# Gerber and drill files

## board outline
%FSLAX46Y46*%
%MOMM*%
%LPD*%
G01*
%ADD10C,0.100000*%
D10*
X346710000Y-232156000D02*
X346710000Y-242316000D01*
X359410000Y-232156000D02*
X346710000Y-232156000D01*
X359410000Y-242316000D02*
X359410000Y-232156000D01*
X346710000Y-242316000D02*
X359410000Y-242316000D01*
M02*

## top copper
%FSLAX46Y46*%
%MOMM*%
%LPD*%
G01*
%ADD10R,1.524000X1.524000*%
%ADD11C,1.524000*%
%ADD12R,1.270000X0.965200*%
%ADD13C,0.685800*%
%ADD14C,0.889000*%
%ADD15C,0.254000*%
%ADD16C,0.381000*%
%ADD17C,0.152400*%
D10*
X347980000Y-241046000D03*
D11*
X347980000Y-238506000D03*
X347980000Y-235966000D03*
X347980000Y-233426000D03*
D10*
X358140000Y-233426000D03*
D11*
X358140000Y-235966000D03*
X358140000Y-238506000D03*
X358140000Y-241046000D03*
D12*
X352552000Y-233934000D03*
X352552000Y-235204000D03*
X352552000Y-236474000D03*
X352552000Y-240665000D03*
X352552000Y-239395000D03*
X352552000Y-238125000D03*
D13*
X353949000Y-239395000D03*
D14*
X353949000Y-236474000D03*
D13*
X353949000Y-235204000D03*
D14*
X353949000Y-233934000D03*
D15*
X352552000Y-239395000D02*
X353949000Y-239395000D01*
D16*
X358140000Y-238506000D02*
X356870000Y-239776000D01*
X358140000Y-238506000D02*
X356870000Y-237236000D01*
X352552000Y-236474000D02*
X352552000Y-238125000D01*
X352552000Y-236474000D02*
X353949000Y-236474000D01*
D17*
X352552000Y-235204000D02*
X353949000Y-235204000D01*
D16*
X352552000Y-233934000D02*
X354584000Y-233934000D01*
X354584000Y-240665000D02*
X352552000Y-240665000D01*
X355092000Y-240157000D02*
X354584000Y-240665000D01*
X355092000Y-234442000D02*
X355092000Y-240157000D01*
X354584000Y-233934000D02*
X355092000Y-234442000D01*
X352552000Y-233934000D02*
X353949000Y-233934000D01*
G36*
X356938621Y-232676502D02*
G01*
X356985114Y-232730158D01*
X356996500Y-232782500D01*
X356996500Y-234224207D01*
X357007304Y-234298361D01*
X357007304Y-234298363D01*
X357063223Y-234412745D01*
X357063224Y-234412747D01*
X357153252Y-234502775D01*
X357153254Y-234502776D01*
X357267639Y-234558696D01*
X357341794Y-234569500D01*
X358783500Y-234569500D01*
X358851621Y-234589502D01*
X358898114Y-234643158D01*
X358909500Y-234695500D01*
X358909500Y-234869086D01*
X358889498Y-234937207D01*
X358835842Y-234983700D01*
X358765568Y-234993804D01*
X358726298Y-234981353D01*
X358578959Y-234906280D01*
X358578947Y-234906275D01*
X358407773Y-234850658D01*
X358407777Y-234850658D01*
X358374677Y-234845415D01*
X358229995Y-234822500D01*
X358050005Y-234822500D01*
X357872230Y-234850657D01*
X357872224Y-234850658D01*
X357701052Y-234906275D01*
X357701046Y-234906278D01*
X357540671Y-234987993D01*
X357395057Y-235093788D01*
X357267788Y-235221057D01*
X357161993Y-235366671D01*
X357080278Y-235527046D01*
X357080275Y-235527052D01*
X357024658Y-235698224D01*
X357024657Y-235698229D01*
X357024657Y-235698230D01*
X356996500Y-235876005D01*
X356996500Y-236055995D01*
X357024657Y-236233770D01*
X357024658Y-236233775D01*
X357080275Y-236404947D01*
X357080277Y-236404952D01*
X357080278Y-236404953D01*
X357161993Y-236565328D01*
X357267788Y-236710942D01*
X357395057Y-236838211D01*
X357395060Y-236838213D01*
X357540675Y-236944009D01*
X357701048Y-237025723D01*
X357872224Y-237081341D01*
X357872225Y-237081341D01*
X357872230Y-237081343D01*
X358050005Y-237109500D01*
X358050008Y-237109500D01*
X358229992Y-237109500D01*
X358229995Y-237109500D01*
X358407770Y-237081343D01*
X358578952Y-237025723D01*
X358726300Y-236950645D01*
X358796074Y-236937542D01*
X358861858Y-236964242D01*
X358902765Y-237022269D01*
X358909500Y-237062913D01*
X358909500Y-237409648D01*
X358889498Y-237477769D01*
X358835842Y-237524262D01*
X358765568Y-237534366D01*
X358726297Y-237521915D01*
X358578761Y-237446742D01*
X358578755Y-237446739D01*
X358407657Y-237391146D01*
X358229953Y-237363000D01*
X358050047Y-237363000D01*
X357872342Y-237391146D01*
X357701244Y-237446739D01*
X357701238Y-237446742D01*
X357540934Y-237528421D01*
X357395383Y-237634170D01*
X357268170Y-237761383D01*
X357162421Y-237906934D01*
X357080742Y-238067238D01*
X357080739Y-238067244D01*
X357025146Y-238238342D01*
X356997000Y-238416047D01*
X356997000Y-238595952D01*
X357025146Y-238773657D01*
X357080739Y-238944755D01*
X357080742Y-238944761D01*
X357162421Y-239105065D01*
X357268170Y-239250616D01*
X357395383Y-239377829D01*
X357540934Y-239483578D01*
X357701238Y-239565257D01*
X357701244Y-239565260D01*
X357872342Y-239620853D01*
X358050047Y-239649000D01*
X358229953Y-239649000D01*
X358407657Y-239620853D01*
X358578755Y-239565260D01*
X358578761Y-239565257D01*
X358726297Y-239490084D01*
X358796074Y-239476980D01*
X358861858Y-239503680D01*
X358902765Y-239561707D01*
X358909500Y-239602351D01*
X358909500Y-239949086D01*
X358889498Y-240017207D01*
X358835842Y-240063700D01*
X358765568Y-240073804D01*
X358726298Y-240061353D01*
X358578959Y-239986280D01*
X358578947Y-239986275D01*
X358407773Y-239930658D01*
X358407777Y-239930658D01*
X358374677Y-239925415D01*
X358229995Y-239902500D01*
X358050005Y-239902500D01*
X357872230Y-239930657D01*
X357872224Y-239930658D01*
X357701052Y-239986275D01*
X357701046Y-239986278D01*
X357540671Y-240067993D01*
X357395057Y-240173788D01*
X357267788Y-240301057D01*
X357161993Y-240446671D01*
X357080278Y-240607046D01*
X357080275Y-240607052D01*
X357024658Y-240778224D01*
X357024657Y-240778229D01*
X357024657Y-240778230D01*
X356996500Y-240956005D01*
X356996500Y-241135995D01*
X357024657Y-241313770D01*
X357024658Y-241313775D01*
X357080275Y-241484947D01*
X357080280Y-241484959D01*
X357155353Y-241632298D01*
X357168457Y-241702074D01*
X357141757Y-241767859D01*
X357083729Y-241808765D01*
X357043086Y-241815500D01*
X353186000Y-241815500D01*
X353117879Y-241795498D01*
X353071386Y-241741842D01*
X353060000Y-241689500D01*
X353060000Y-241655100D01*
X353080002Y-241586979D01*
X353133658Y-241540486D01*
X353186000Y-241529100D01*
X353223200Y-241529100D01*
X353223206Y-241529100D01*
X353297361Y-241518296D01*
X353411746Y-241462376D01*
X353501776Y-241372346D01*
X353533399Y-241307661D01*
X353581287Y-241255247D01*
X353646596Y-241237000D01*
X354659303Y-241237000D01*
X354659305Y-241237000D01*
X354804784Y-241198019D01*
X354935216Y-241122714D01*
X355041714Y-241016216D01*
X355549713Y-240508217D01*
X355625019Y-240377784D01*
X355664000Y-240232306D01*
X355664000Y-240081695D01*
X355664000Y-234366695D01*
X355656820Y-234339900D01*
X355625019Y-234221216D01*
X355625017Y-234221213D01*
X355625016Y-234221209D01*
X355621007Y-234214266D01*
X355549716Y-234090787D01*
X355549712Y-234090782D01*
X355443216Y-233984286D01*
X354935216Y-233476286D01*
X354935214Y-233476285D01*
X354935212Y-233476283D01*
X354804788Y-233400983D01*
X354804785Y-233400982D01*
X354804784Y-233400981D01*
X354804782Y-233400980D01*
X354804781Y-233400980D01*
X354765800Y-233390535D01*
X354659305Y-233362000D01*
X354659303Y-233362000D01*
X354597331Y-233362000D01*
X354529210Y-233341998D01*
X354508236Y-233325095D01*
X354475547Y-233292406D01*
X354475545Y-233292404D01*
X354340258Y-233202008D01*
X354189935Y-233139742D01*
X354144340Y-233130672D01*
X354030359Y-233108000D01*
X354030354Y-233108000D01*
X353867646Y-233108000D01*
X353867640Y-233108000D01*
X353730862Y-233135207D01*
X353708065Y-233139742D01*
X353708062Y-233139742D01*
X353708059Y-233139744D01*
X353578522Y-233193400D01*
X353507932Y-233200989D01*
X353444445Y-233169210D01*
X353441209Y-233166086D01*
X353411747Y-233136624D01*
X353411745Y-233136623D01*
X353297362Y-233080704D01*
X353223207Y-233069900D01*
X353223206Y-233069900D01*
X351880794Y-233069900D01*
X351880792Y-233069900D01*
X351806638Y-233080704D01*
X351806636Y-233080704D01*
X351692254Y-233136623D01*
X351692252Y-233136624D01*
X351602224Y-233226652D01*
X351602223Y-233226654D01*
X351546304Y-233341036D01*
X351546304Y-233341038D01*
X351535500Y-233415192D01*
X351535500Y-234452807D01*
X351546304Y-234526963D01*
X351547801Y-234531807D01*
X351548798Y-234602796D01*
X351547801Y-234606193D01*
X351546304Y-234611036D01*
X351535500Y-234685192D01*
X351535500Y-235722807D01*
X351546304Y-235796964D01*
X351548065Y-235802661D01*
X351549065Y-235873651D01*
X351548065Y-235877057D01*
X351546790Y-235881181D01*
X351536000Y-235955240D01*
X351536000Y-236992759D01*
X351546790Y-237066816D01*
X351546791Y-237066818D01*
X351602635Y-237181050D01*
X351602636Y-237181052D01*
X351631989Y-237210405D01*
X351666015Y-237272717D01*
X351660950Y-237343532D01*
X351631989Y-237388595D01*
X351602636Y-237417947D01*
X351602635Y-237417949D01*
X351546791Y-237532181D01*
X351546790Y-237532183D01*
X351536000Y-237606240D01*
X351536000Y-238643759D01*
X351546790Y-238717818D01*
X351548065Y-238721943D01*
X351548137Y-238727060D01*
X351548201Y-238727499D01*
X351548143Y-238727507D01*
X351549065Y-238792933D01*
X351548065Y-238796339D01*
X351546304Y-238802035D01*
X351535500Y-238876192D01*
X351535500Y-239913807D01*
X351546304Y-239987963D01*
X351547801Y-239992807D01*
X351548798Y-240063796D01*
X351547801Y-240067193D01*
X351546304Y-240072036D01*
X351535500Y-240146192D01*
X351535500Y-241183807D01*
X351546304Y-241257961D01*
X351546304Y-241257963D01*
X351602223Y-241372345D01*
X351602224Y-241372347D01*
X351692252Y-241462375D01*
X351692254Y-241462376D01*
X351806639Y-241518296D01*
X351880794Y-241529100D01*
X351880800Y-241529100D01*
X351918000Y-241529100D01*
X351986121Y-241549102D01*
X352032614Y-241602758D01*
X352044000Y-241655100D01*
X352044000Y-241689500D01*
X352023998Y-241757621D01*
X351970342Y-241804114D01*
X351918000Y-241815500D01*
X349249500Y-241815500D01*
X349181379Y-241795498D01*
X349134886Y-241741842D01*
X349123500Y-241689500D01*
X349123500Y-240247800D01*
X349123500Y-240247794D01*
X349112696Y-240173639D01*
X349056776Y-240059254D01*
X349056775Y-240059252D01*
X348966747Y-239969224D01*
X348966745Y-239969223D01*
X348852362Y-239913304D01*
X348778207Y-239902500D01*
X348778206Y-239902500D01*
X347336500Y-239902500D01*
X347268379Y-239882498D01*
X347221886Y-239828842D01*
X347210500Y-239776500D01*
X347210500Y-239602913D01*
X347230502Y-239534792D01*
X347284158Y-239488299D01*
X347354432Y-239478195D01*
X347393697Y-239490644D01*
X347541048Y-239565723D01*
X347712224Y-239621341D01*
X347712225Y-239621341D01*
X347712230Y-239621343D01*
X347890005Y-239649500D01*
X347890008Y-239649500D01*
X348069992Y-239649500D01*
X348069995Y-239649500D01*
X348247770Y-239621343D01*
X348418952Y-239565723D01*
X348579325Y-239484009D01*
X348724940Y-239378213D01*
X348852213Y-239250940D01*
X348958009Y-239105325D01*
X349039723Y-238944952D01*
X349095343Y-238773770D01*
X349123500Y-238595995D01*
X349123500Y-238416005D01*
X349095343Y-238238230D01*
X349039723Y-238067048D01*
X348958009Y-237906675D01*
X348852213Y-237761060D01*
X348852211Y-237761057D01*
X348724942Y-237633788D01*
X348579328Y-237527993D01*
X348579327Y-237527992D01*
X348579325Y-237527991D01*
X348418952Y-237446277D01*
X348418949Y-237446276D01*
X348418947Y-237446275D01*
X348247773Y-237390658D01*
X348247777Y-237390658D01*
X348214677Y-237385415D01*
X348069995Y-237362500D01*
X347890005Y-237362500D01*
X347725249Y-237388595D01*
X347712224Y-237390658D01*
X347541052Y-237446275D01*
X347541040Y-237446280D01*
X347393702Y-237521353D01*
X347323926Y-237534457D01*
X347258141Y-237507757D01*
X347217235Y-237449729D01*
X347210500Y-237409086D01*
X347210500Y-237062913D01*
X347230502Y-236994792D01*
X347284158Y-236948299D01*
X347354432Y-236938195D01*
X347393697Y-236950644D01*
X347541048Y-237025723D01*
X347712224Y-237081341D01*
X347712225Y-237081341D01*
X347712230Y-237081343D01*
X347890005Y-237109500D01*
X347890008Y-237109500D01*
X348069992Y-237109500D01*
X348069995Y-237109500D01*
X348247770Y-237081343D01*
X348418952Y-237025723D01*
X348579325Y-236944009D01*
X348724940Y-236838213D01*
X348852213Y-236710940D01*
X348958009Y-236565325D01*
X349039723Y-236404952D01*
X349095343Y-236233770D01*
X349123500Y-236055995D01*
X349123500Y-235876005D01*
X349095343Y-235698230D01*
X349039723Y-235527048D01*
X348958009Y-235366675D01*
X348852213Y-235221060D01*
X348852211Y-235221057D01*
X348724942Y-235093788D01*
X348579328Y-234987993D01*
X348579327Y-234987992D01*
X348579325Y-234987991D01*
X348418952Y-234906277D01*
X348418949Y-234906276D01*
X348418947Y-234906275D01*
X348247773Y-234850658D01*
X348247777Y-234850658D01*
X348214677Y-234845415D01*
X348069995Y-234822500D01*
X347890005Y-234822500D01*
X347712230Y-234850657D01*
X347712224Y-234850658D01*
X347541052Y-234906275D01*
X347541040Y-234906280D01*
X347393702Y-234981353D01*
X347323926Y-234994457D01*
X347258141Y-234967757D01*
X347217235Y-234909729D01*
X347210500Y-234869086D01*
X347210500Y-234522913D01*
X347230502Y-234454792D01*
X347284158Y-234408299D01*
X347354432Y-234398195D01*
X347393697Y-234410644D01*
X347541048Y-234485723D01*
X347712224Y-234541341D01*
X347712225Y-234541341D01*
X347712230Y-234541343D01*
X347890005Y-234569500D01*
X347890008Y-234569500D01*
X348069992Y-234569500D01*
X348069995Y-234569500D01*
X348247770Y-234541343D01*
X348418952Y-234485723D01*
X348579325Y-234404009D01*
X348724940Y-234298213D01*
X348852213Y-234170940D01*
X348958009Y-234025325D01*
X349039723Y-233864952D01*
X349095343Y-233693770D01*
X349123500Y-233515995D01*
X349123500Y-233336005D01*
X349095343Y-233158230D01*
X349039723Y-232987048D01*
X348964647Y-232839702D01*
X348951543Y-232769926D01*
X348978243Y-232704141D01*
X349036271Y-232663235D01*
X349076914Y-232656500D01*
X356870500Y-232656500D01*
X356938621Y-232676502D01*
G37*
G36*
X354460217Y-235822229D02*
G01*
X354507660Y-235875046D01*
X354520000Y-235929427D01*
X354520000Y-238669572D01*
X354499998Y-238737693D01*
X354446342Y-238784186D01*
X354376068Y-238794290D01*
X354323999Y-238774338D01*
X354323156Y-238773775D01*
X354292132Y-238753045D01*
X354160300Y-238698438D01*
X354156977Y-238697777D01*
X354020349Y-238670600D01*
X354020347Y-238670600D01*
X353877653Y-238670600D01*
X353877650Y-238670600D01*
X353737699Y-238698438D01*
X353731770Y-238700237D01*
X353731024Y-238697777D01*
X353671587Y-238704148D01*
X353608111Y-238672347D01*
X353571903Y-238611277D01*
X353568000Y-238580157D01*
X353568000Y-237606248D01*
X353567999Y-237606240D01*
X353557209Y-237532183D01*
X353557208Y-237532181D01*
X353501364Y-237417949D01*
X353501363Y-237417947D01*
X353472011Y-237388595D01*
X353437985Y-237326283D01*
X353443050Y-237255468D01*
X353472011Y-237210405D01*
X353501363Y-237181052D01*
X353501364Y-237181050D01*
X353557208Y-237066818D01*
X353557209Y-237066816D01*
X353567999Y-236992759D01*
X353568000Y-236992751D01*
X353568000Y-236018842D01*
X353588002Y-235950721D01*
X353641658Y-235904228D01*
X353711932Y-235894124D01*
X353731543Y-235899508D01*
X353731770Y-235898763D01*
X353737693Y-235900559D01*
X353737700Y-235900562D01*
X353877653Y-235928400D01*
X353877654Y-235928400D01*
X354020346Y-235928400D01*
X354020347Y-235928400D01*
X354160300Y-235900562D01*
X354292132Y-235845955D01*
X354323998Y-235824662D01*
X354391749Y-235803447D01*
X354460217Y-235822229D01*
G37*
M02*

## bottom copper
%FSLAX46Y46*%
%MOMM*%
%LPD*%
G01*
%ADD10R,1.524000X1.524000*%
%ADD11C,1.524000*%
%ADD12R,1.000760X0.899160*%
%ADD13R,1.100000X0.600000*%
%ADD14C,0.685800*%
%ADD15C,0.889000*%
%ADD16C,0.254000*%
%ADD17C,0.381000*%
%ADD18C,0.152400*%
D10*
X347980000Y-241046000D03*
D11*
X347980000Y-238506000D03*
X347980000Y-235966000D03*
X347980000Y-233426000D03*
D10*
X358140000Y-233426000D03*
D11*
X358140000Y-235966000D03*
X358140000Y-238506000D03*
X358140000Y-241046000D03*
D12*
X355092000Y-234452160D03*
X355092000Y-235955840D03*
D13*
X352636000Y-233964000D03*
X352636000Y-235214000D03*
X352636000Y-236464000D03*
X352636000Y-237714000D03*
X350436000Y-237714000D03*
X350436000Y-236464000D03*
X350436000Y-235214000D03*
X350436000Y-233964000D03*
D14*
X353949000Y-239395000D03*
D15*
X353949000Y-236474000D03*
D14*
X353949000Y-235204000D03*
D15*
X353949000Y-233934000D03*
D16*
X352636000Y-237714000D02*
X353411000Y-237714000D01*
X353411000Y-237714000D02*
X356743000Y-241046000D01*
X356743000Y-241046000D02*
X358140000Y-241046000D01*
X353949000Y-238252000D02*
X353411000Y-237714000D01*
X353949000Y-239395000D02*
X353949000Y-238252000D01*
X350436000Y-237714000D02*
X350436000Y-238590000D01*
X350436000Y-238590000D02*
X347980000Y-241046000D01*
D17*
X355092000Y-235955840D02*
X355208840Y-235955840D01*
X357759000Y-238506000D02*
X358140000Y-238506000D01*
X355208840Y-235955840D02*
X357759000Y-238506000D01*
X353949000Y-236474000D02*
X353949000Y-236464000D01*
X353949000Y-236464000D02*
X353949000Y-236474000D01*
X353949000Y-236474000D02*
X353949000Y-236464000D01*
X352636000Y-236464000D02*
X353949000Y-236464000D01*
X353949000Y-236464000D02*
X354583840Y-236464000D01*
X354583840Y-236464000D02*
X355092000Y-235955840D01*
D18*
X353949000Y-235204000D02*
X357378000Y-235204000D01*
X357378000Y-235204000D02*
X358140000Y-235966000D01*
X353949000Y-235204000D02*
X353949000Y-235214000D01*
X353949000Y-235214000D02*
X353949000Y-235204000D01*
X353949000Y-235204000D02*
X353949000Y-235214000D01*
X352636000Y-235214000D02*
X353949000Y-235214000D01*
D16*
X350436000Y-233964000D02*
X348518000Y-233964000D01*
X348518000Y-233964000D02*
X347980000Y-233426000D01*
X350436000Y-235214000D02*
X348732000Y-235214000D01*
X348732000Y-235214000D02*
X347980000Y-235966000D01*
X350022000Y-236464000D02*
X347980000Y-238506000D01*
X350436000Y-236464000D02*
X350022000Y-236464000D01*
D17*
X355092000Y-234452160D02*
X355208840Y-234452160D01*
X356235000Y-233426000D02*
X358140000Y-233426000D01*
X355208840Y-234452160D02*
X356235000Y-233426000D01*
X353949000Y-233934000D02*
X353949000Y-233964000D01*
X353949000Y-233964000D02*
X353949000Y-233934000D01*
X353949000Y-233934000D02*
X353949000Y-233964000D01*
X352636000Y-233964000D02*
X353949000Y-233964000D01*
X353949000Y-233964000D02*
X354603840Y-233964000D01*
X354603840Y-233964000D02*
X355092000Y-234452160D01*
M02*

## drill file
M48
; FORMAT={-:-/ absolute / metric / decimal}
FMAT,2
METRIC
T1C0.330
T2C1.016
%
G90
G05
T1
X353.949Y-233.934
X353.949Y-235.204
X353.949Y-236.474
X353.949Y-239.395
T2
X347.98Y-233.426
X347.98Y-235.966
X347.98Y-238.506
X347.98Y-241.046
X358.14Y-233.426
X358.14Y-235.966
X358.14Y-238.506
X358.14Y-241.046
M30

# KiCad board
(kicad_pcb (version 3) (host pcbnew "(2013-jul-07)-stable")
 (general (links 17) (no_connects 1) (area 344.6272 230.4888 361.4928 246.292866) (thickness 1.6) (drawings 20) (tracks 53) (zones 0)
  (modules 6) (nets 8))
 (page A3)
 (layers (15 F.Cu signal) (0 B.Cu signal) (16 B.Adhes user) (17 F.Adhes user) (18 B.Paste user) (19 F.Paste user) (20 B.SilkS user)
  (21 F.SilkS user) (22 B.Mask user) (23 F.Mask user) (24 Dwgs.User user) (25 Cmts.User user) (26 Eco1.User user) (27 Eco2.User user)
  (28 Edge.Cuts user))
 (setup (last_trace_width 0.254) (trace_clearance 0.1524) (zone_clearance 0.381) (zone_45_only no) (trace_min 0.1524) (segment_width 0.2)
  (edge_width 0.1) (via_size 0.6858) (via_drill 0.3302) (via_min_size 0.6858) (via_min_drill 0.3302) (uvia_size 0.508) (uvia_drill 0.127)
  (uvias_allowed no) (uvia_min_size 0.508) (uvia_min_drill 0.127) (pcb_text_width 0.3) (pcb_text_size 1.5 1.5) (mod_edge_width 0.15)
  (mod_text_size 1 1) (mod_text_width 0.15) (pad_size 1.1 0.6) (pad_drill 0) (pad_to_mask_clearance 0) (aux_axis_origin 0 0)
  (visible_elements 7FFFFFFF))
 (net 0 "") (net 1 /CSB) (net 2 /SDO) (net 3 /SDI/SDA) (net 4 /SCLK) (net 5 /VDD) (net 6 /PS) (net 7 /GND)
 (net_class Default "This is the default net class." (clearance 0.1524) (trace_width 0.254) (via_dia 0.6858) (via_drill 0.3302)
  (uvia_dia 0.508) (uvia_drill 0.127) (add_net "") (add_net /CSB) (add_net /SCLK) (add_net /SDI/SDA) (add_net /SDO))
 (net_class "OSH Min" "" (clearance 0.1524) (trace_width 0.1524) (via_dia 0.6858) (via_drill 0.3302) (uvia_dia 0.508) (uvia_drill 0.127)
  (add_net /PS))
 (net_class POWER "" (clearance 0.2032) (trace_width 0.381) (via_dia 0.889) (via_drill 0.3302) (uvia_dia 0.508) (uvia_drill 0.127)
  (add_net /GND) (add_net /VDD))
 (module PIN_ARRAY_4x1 (layer B.Cu) (at 347.98 237.236 90)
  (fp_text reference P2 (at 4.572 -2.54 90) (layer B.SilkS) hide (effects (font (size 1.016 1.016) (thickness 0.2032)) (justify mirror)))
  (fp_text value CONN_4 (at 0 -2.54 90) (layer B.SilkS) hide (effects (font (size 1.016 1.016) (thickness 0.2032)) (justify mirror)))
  (pad 1 thru_hole rect (at -3.81 0 90) (size 1.524 1.524) (drill 1.016) (layers *.Cu *.Mask B.SilkS) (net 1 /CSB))
  (pad 2 thru_hole circle (at -1.27 0 90) (size 1.524 1.524) (drill 1.016) (layers *.Cu *.Mask B.SilkS) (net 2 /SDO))
  (pad 3 thru_hole circle (at 1.27 0 90) (size 1.524 1.524) (drill 1.016) (layers *.Cu *.Mask B.SilkS) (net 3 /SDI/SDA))
  (pad 4 thru_hole circle (at 3.81 0 90) (size 1.524 1.524) (drill 1.016) (layers *.Cu *.Mask B.SilkS) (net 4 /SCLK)))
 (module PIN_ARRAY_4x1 (layer B.Cu) (at 358.14 237.236 270)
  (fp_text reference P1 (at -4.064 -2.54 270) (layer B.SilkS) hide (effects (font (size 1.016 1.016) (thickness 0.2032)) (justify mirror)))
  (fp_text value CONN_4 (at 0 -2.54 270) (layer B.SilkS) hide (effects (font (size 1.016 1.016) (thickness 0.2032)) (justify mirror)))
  (pad 1 thru_hole rect (at -3.81 0 270) (size 1.524 1.524) (drill 1.016) (layers *.Cu *.Mask B.SilkS) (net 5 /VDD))
  (pad 2 thru_hole circle (at -1.27 0 270) (size 1.524 1.524) (drill 1.016) (layers *.Cu *.Mask B.SilkS) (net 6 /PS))
  (pad 3 thru_hole circle (at 1.27 0 270) (size 1.524 1.524) (drill 1.016) (layers *.Cu *.Mask B.SilkS) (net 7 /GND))
  (pad 4 thru_hole circle (at 3.81 0 270) (size 1.524 1.524) (drill 1.016) (layers *.Cu *.Mask B.SilkS) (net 1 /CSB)))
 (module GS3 (layer F.Cu) (at 352.552 235.204)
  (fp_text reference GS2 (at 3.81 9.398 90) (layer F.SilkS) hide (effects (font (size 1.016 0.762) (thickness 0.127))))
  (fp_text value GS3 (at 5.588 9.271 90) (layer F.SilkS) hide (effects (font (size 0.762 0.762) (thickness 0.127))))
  (pad 1 smd rect (at 0 -1.27) (size 1.27 0.9652) (layers F.Cu F.Paste F.Mask) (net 5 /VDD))
  (pad 2 smd rect (at 0 0) (size 1.27 0.9652) (layers F.Cu F.Paste F.Mask) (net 6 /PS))
  (pad 3 smd rect (at 0 1.27) (size 1.27 0.9652) (layers F.Cu F.Paste F.Mask) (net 7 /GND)))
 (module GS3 (layer F.Cu) (at 352.552 239.395 180)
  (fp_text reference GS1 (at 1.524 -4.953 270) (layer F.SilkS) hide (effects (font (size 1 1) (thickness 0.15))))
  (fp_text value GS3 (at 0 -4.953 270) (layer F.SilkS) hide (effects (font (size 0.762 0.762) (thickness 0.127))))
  (pad 1 smd rect (at 0 -1.27 180) (size 1.27 0.9652) (layers F.Cu F.Paste F.Mask) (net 5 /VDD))
  (pad 2 smd rect (at 0 0 180) (size 1.27 0.9652) (layers F.Cu F.Paste F.Mask) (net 1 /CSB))
  (pad 3 smd rect (at 0 1.27 180) (size 1.27 0.9652) (layers F.Cu F.Paste F.Mask) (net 7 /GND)))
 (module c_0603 (layer B.Cu) (at 355.092 235.204 90)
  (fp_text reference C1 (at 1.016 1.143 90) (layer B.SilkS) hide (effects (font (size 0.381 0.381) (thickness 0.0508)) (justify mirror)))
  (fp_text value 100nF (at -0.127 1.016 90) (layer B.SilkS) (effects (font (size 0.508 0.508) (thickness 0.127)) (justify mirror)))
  (pad 1 smd rect (at 0.75184 0 90) (size 0.89916 1.00076) (layers B.Cu B.Paste B.Mask) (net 5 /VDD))
  (pad 2 smd rect (at -0.75184 0 90) (size 0.89916 1.00076) (layers B.Cu B.Paste B.Mask) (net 7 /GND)))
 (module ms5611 (layer B.Cu) (at 351.536 235.839 180)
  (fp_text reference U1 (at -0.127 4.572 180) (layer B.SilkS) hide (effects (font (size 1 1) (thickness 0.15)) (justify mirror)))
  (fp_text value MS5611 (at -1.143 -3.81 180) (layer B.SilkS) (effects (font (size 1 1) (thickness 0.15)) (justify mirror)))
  (pad 1 smd rect (at -1.1 1.875 180) (size 1.1 0.6) (layers B.Cu B.Paste B.Mask) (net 5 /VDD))
  (pad 2 smd rect (at -1.1 0.625 180) (size 1.1 0.6) (layers B.Cu B.Paste B.Mask) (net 6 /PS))
  (pad 3 smd rect (at -1.1 -0.625 180) (size 1.1 0.6) (layers B.Cu B.Paste B.Mask) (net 7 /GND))
  (pad 4 smd rect (at -1.1 -1.875 180) (size 1.1 0.6) (layers B.Cu B.Paste B.Mask) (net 1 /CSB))
  (pad 5 smd rect (at 1.1 -1.875 180) (size 1.1 0.6) (layers B.Cu B.Paste B.Mask) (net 1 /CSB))
  (pad 6 smd rect (at 1.1 -0.625 180) (size 1.1 0.6) (layers B.Cu B.Paste B.Mask) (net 2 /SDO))
  (pad 7 smd rect (at 1.1 0.625 180) (size 1.1 0.6) (layers B.Cu B.Paste B.Mask) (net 3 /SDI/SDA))
  (pad 8 smd rect (at 1.1 1.875 180) (size 1.1 0.6) (layers B.Cu B.Paste B.Mask) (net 4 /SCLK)))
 (gr_line (start 346.71 232.156) (end 346.71 242.316) (angle 90) (layer Edge.Cuts) (width 0.1))
 (gr_line (start 359.41 232.156) (end 346.71 232.156) (angle 90) (layer Edge.Cuts) (width 0.1))
 (gr_line (start 359.41 242.316) (end 359.41 232.156) (angle 90) (layer Edge.Cuts) (width 0.1))
 (gr_line (start 346.71 242.316) (end 359.41 242.316) (angle 90) (layer Edge.Cuts) (width 0.1))
 (segment (start 352.636 237.714) (end 353.411 237.714) (width 0.254) (layer B.Cu) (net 1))
 (segment (start 353.411 237.714) (end 356.743 241.046) (width 0.254) (layer B.Cu) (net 1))
 (segment (start 356.743 241.046) (end 358.14 241.046) (width 0.254) (layer B.Cu) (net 1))
 (segment (start 352.552 239.395) (end 353.949 239.395) (width 0.254) (layer F.Cu) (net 1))
 (segment (start 353.949 238.252) (end 353.411 237.714) (width 0.254) (layer B.Cu) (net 1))
 (segment (start 353.949 239.395) (end 353.949 238.252) (width 0.254) (layer B.Cu) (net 1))
 (via (at 353.949 239.395) (size 0.6858) (layers F.Cu B.Cu) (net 1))
 (segment (start 350.436 237.714) (end 350.436 238.59) (width 0.254) (layer B.Cu) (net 1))
 (segment (start 350.436 238.59) (end 347.98 241.046) (width 0.254) (layer B.Cu) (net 1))
 (segment (start 358.14 238.506) (end 356.87 239.776) (width 0.381) (layer F.Cu) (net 7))
 (segment (start 358.14 238.506) (end 356.87 237.236) (width 0.381) (layer F.Cu) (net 7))
 (segment (start 352.552 236.474) (end 352.552 238.125) (width 0.381) (layer F.Cu) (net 7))
 (segment (start 355.092 235.95584) (end 355.20884 235.95584) (width 0.381) (layer B.Cu) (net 7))
 (segment (start 357.759 238.506) (end 358.14 238.506) (width 0.381) (layer B.Cu) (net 7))
 (segment (start 355.20884 235.95584) (end 357.759 238.506) (width 0.381) (layer B.Cu) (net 7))
 (segment (start 352.552 236.474) (end 353.949 236.474) (width 0.381) (layer F.Cu) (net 7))
 (via (at 353.949 236.474) (size 0.889) (layers F.Cu B.Cu) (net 7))
 (segment (start 353.949 236.474) (end 353.949 236.464) (width 0.381) (layer B.Cu) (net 7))
 (segment (start 353.949 236.464) (end 353.949 236.474) (width 0.381) (layer B.Cu) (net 7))
 (segment (start 353.949 236.474) (end 353.949 236.464) (width 0.381) (layer B.Cu) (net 7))
 (segment (start 352.636 236.464) (end 353.949 236.464) (width 0.381) (layer B.Cu) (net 7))
 (segment (start 353.949 236.464) (end 354.58384 236.464) (width 0.381) (layer B.Cu) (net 7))
 (segment (start 354.58384 236.464) (end 355.092 235.95584) (width 0.381) (layer B.Cu) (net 7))
 (segment (start 353.949 235.204) (end 357.378 235.204) (width 0.1524) (layer B.Cu) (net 6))
 (segment (start 357.378 235.204) (end 358.14 235.966) (width 0.1524) (layer B.Cu) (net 6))
 (segment (start 352.552 235.204) (end 353.949 235.204) (width 0.1524) (layer F.Cu) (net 6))
 (via (at 353.949 235.204) (size 0.6858) (layers F.Cu B.Cu) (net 6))
 (segment (start 353.949 235.204) (end 353.949 235.214) (width 0.1524) (layer B.Cu) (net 6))
 (segment (start 353.949 235.214) (end 353.949 235.204) (width 0.1524) (layer B.Cu) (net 6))
 (segment (start 353.949 235.204) (end 353.949 235.214) (width 0.1524) (layer B.Cu) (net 6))
 (segment (start 352.636 235.214) (end 353.949 235.214) (width 0.1524) (layer B.Cu) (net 6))
 (segment (start 350.436 233.964) (end 348.518 233.964) (width 0.254) (layer B.Cu) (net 4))
 (segment (start 348.518 233.964) (end 347.98 233.426) (width 0.254) (layer B.Cu) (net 4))
 (segment (start 350.436 235.214) (end 348.732 235.214) (width 0.254) (layer B.Cu) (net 3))
 (segment (start 348.732 235.214) (end 347.98 235.966) (width 0.254) (layer B.Cu) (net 3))
 (segment (start 350.022 236.464) (end 347.98 238.506) (width 0.254) (layer B.Cu) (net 2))
 (segment (start 350.436 236.464) (end 350.022 236.464) (width 0.254) (layer B.Cu) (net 2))
 (segment (start 352.552 233.934) (end 354.584 233.934) (width 0.381) (layer F.Cu) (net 5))
 (segment (start 354.584 240.665) (end 352.552 240.665) (width 0.381) (layer F.Cu) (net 5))
 (segment (start 355.092 240.157) (end 354.584 240.665) (width 0.381) (layer F.Cu) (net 5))
 (segment (start 355.092 234.442) (end 355.092 240.157) (width 0.381) (layer F.Cu) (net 5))
 (segment (start 354.584 233.934) (end 355.092 234.442) (width 0.381) (layer F.Cu) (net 5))
 (segment (start 355.092 234.45216) (end 355.20884 234.45216) (width 0.381) (layer B.Cu) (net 5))
 (segment (start 356.235 233.426) (end 358.14 233.426) (width 0.381) (layer B.Cu) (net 5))
 (segment (start 355.20884 234.45216) (end 356.235 233.426) (width 0.381) (layer B.Cu) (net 5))
 (segment (start 352.552 233.934) (end 353.949 233.934) (width 0.381) (layer F.Cu) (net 5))
 (via (at 353.949 233.934) (size 0.889) (layers F.Cu B.Cu) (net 5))
 (segment (start 353.949 233.934) (end 353.949 233.964) (width 0.381) (layer B.Cu) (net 5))
 (segment (start 353.949 233.964) (end 353.949 233.934) (width 0.381) (layer B.Cu) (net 5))
 (segment (start 353.949 233.934) (end 353.949 233.964) (width 0.381) (layer B.Cu) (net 5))
 (segment (start 352.636 233.964) (end 353.949 233.964) (width 0.381) (layer B.Cu) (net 5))
 (segment (start 353.949 233.964) (end 354.60384 233.964) (width 0.381) (layer B.Cu) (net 5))
 (segment (start 354.60384 233.964) (end 355.092 234.45216) (width 0.381) (layer B.Cu) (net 5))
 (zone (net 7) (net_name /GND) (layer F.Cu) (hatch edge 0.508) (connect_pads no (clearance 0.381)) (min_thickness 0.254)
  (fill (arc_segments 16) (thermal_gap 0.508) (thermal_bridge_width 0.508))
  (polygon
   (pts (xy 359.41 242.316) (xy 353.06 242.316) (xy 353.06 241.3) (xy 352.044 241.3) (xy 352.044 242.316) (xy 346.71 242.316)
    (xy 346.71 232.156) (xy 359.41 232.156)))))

